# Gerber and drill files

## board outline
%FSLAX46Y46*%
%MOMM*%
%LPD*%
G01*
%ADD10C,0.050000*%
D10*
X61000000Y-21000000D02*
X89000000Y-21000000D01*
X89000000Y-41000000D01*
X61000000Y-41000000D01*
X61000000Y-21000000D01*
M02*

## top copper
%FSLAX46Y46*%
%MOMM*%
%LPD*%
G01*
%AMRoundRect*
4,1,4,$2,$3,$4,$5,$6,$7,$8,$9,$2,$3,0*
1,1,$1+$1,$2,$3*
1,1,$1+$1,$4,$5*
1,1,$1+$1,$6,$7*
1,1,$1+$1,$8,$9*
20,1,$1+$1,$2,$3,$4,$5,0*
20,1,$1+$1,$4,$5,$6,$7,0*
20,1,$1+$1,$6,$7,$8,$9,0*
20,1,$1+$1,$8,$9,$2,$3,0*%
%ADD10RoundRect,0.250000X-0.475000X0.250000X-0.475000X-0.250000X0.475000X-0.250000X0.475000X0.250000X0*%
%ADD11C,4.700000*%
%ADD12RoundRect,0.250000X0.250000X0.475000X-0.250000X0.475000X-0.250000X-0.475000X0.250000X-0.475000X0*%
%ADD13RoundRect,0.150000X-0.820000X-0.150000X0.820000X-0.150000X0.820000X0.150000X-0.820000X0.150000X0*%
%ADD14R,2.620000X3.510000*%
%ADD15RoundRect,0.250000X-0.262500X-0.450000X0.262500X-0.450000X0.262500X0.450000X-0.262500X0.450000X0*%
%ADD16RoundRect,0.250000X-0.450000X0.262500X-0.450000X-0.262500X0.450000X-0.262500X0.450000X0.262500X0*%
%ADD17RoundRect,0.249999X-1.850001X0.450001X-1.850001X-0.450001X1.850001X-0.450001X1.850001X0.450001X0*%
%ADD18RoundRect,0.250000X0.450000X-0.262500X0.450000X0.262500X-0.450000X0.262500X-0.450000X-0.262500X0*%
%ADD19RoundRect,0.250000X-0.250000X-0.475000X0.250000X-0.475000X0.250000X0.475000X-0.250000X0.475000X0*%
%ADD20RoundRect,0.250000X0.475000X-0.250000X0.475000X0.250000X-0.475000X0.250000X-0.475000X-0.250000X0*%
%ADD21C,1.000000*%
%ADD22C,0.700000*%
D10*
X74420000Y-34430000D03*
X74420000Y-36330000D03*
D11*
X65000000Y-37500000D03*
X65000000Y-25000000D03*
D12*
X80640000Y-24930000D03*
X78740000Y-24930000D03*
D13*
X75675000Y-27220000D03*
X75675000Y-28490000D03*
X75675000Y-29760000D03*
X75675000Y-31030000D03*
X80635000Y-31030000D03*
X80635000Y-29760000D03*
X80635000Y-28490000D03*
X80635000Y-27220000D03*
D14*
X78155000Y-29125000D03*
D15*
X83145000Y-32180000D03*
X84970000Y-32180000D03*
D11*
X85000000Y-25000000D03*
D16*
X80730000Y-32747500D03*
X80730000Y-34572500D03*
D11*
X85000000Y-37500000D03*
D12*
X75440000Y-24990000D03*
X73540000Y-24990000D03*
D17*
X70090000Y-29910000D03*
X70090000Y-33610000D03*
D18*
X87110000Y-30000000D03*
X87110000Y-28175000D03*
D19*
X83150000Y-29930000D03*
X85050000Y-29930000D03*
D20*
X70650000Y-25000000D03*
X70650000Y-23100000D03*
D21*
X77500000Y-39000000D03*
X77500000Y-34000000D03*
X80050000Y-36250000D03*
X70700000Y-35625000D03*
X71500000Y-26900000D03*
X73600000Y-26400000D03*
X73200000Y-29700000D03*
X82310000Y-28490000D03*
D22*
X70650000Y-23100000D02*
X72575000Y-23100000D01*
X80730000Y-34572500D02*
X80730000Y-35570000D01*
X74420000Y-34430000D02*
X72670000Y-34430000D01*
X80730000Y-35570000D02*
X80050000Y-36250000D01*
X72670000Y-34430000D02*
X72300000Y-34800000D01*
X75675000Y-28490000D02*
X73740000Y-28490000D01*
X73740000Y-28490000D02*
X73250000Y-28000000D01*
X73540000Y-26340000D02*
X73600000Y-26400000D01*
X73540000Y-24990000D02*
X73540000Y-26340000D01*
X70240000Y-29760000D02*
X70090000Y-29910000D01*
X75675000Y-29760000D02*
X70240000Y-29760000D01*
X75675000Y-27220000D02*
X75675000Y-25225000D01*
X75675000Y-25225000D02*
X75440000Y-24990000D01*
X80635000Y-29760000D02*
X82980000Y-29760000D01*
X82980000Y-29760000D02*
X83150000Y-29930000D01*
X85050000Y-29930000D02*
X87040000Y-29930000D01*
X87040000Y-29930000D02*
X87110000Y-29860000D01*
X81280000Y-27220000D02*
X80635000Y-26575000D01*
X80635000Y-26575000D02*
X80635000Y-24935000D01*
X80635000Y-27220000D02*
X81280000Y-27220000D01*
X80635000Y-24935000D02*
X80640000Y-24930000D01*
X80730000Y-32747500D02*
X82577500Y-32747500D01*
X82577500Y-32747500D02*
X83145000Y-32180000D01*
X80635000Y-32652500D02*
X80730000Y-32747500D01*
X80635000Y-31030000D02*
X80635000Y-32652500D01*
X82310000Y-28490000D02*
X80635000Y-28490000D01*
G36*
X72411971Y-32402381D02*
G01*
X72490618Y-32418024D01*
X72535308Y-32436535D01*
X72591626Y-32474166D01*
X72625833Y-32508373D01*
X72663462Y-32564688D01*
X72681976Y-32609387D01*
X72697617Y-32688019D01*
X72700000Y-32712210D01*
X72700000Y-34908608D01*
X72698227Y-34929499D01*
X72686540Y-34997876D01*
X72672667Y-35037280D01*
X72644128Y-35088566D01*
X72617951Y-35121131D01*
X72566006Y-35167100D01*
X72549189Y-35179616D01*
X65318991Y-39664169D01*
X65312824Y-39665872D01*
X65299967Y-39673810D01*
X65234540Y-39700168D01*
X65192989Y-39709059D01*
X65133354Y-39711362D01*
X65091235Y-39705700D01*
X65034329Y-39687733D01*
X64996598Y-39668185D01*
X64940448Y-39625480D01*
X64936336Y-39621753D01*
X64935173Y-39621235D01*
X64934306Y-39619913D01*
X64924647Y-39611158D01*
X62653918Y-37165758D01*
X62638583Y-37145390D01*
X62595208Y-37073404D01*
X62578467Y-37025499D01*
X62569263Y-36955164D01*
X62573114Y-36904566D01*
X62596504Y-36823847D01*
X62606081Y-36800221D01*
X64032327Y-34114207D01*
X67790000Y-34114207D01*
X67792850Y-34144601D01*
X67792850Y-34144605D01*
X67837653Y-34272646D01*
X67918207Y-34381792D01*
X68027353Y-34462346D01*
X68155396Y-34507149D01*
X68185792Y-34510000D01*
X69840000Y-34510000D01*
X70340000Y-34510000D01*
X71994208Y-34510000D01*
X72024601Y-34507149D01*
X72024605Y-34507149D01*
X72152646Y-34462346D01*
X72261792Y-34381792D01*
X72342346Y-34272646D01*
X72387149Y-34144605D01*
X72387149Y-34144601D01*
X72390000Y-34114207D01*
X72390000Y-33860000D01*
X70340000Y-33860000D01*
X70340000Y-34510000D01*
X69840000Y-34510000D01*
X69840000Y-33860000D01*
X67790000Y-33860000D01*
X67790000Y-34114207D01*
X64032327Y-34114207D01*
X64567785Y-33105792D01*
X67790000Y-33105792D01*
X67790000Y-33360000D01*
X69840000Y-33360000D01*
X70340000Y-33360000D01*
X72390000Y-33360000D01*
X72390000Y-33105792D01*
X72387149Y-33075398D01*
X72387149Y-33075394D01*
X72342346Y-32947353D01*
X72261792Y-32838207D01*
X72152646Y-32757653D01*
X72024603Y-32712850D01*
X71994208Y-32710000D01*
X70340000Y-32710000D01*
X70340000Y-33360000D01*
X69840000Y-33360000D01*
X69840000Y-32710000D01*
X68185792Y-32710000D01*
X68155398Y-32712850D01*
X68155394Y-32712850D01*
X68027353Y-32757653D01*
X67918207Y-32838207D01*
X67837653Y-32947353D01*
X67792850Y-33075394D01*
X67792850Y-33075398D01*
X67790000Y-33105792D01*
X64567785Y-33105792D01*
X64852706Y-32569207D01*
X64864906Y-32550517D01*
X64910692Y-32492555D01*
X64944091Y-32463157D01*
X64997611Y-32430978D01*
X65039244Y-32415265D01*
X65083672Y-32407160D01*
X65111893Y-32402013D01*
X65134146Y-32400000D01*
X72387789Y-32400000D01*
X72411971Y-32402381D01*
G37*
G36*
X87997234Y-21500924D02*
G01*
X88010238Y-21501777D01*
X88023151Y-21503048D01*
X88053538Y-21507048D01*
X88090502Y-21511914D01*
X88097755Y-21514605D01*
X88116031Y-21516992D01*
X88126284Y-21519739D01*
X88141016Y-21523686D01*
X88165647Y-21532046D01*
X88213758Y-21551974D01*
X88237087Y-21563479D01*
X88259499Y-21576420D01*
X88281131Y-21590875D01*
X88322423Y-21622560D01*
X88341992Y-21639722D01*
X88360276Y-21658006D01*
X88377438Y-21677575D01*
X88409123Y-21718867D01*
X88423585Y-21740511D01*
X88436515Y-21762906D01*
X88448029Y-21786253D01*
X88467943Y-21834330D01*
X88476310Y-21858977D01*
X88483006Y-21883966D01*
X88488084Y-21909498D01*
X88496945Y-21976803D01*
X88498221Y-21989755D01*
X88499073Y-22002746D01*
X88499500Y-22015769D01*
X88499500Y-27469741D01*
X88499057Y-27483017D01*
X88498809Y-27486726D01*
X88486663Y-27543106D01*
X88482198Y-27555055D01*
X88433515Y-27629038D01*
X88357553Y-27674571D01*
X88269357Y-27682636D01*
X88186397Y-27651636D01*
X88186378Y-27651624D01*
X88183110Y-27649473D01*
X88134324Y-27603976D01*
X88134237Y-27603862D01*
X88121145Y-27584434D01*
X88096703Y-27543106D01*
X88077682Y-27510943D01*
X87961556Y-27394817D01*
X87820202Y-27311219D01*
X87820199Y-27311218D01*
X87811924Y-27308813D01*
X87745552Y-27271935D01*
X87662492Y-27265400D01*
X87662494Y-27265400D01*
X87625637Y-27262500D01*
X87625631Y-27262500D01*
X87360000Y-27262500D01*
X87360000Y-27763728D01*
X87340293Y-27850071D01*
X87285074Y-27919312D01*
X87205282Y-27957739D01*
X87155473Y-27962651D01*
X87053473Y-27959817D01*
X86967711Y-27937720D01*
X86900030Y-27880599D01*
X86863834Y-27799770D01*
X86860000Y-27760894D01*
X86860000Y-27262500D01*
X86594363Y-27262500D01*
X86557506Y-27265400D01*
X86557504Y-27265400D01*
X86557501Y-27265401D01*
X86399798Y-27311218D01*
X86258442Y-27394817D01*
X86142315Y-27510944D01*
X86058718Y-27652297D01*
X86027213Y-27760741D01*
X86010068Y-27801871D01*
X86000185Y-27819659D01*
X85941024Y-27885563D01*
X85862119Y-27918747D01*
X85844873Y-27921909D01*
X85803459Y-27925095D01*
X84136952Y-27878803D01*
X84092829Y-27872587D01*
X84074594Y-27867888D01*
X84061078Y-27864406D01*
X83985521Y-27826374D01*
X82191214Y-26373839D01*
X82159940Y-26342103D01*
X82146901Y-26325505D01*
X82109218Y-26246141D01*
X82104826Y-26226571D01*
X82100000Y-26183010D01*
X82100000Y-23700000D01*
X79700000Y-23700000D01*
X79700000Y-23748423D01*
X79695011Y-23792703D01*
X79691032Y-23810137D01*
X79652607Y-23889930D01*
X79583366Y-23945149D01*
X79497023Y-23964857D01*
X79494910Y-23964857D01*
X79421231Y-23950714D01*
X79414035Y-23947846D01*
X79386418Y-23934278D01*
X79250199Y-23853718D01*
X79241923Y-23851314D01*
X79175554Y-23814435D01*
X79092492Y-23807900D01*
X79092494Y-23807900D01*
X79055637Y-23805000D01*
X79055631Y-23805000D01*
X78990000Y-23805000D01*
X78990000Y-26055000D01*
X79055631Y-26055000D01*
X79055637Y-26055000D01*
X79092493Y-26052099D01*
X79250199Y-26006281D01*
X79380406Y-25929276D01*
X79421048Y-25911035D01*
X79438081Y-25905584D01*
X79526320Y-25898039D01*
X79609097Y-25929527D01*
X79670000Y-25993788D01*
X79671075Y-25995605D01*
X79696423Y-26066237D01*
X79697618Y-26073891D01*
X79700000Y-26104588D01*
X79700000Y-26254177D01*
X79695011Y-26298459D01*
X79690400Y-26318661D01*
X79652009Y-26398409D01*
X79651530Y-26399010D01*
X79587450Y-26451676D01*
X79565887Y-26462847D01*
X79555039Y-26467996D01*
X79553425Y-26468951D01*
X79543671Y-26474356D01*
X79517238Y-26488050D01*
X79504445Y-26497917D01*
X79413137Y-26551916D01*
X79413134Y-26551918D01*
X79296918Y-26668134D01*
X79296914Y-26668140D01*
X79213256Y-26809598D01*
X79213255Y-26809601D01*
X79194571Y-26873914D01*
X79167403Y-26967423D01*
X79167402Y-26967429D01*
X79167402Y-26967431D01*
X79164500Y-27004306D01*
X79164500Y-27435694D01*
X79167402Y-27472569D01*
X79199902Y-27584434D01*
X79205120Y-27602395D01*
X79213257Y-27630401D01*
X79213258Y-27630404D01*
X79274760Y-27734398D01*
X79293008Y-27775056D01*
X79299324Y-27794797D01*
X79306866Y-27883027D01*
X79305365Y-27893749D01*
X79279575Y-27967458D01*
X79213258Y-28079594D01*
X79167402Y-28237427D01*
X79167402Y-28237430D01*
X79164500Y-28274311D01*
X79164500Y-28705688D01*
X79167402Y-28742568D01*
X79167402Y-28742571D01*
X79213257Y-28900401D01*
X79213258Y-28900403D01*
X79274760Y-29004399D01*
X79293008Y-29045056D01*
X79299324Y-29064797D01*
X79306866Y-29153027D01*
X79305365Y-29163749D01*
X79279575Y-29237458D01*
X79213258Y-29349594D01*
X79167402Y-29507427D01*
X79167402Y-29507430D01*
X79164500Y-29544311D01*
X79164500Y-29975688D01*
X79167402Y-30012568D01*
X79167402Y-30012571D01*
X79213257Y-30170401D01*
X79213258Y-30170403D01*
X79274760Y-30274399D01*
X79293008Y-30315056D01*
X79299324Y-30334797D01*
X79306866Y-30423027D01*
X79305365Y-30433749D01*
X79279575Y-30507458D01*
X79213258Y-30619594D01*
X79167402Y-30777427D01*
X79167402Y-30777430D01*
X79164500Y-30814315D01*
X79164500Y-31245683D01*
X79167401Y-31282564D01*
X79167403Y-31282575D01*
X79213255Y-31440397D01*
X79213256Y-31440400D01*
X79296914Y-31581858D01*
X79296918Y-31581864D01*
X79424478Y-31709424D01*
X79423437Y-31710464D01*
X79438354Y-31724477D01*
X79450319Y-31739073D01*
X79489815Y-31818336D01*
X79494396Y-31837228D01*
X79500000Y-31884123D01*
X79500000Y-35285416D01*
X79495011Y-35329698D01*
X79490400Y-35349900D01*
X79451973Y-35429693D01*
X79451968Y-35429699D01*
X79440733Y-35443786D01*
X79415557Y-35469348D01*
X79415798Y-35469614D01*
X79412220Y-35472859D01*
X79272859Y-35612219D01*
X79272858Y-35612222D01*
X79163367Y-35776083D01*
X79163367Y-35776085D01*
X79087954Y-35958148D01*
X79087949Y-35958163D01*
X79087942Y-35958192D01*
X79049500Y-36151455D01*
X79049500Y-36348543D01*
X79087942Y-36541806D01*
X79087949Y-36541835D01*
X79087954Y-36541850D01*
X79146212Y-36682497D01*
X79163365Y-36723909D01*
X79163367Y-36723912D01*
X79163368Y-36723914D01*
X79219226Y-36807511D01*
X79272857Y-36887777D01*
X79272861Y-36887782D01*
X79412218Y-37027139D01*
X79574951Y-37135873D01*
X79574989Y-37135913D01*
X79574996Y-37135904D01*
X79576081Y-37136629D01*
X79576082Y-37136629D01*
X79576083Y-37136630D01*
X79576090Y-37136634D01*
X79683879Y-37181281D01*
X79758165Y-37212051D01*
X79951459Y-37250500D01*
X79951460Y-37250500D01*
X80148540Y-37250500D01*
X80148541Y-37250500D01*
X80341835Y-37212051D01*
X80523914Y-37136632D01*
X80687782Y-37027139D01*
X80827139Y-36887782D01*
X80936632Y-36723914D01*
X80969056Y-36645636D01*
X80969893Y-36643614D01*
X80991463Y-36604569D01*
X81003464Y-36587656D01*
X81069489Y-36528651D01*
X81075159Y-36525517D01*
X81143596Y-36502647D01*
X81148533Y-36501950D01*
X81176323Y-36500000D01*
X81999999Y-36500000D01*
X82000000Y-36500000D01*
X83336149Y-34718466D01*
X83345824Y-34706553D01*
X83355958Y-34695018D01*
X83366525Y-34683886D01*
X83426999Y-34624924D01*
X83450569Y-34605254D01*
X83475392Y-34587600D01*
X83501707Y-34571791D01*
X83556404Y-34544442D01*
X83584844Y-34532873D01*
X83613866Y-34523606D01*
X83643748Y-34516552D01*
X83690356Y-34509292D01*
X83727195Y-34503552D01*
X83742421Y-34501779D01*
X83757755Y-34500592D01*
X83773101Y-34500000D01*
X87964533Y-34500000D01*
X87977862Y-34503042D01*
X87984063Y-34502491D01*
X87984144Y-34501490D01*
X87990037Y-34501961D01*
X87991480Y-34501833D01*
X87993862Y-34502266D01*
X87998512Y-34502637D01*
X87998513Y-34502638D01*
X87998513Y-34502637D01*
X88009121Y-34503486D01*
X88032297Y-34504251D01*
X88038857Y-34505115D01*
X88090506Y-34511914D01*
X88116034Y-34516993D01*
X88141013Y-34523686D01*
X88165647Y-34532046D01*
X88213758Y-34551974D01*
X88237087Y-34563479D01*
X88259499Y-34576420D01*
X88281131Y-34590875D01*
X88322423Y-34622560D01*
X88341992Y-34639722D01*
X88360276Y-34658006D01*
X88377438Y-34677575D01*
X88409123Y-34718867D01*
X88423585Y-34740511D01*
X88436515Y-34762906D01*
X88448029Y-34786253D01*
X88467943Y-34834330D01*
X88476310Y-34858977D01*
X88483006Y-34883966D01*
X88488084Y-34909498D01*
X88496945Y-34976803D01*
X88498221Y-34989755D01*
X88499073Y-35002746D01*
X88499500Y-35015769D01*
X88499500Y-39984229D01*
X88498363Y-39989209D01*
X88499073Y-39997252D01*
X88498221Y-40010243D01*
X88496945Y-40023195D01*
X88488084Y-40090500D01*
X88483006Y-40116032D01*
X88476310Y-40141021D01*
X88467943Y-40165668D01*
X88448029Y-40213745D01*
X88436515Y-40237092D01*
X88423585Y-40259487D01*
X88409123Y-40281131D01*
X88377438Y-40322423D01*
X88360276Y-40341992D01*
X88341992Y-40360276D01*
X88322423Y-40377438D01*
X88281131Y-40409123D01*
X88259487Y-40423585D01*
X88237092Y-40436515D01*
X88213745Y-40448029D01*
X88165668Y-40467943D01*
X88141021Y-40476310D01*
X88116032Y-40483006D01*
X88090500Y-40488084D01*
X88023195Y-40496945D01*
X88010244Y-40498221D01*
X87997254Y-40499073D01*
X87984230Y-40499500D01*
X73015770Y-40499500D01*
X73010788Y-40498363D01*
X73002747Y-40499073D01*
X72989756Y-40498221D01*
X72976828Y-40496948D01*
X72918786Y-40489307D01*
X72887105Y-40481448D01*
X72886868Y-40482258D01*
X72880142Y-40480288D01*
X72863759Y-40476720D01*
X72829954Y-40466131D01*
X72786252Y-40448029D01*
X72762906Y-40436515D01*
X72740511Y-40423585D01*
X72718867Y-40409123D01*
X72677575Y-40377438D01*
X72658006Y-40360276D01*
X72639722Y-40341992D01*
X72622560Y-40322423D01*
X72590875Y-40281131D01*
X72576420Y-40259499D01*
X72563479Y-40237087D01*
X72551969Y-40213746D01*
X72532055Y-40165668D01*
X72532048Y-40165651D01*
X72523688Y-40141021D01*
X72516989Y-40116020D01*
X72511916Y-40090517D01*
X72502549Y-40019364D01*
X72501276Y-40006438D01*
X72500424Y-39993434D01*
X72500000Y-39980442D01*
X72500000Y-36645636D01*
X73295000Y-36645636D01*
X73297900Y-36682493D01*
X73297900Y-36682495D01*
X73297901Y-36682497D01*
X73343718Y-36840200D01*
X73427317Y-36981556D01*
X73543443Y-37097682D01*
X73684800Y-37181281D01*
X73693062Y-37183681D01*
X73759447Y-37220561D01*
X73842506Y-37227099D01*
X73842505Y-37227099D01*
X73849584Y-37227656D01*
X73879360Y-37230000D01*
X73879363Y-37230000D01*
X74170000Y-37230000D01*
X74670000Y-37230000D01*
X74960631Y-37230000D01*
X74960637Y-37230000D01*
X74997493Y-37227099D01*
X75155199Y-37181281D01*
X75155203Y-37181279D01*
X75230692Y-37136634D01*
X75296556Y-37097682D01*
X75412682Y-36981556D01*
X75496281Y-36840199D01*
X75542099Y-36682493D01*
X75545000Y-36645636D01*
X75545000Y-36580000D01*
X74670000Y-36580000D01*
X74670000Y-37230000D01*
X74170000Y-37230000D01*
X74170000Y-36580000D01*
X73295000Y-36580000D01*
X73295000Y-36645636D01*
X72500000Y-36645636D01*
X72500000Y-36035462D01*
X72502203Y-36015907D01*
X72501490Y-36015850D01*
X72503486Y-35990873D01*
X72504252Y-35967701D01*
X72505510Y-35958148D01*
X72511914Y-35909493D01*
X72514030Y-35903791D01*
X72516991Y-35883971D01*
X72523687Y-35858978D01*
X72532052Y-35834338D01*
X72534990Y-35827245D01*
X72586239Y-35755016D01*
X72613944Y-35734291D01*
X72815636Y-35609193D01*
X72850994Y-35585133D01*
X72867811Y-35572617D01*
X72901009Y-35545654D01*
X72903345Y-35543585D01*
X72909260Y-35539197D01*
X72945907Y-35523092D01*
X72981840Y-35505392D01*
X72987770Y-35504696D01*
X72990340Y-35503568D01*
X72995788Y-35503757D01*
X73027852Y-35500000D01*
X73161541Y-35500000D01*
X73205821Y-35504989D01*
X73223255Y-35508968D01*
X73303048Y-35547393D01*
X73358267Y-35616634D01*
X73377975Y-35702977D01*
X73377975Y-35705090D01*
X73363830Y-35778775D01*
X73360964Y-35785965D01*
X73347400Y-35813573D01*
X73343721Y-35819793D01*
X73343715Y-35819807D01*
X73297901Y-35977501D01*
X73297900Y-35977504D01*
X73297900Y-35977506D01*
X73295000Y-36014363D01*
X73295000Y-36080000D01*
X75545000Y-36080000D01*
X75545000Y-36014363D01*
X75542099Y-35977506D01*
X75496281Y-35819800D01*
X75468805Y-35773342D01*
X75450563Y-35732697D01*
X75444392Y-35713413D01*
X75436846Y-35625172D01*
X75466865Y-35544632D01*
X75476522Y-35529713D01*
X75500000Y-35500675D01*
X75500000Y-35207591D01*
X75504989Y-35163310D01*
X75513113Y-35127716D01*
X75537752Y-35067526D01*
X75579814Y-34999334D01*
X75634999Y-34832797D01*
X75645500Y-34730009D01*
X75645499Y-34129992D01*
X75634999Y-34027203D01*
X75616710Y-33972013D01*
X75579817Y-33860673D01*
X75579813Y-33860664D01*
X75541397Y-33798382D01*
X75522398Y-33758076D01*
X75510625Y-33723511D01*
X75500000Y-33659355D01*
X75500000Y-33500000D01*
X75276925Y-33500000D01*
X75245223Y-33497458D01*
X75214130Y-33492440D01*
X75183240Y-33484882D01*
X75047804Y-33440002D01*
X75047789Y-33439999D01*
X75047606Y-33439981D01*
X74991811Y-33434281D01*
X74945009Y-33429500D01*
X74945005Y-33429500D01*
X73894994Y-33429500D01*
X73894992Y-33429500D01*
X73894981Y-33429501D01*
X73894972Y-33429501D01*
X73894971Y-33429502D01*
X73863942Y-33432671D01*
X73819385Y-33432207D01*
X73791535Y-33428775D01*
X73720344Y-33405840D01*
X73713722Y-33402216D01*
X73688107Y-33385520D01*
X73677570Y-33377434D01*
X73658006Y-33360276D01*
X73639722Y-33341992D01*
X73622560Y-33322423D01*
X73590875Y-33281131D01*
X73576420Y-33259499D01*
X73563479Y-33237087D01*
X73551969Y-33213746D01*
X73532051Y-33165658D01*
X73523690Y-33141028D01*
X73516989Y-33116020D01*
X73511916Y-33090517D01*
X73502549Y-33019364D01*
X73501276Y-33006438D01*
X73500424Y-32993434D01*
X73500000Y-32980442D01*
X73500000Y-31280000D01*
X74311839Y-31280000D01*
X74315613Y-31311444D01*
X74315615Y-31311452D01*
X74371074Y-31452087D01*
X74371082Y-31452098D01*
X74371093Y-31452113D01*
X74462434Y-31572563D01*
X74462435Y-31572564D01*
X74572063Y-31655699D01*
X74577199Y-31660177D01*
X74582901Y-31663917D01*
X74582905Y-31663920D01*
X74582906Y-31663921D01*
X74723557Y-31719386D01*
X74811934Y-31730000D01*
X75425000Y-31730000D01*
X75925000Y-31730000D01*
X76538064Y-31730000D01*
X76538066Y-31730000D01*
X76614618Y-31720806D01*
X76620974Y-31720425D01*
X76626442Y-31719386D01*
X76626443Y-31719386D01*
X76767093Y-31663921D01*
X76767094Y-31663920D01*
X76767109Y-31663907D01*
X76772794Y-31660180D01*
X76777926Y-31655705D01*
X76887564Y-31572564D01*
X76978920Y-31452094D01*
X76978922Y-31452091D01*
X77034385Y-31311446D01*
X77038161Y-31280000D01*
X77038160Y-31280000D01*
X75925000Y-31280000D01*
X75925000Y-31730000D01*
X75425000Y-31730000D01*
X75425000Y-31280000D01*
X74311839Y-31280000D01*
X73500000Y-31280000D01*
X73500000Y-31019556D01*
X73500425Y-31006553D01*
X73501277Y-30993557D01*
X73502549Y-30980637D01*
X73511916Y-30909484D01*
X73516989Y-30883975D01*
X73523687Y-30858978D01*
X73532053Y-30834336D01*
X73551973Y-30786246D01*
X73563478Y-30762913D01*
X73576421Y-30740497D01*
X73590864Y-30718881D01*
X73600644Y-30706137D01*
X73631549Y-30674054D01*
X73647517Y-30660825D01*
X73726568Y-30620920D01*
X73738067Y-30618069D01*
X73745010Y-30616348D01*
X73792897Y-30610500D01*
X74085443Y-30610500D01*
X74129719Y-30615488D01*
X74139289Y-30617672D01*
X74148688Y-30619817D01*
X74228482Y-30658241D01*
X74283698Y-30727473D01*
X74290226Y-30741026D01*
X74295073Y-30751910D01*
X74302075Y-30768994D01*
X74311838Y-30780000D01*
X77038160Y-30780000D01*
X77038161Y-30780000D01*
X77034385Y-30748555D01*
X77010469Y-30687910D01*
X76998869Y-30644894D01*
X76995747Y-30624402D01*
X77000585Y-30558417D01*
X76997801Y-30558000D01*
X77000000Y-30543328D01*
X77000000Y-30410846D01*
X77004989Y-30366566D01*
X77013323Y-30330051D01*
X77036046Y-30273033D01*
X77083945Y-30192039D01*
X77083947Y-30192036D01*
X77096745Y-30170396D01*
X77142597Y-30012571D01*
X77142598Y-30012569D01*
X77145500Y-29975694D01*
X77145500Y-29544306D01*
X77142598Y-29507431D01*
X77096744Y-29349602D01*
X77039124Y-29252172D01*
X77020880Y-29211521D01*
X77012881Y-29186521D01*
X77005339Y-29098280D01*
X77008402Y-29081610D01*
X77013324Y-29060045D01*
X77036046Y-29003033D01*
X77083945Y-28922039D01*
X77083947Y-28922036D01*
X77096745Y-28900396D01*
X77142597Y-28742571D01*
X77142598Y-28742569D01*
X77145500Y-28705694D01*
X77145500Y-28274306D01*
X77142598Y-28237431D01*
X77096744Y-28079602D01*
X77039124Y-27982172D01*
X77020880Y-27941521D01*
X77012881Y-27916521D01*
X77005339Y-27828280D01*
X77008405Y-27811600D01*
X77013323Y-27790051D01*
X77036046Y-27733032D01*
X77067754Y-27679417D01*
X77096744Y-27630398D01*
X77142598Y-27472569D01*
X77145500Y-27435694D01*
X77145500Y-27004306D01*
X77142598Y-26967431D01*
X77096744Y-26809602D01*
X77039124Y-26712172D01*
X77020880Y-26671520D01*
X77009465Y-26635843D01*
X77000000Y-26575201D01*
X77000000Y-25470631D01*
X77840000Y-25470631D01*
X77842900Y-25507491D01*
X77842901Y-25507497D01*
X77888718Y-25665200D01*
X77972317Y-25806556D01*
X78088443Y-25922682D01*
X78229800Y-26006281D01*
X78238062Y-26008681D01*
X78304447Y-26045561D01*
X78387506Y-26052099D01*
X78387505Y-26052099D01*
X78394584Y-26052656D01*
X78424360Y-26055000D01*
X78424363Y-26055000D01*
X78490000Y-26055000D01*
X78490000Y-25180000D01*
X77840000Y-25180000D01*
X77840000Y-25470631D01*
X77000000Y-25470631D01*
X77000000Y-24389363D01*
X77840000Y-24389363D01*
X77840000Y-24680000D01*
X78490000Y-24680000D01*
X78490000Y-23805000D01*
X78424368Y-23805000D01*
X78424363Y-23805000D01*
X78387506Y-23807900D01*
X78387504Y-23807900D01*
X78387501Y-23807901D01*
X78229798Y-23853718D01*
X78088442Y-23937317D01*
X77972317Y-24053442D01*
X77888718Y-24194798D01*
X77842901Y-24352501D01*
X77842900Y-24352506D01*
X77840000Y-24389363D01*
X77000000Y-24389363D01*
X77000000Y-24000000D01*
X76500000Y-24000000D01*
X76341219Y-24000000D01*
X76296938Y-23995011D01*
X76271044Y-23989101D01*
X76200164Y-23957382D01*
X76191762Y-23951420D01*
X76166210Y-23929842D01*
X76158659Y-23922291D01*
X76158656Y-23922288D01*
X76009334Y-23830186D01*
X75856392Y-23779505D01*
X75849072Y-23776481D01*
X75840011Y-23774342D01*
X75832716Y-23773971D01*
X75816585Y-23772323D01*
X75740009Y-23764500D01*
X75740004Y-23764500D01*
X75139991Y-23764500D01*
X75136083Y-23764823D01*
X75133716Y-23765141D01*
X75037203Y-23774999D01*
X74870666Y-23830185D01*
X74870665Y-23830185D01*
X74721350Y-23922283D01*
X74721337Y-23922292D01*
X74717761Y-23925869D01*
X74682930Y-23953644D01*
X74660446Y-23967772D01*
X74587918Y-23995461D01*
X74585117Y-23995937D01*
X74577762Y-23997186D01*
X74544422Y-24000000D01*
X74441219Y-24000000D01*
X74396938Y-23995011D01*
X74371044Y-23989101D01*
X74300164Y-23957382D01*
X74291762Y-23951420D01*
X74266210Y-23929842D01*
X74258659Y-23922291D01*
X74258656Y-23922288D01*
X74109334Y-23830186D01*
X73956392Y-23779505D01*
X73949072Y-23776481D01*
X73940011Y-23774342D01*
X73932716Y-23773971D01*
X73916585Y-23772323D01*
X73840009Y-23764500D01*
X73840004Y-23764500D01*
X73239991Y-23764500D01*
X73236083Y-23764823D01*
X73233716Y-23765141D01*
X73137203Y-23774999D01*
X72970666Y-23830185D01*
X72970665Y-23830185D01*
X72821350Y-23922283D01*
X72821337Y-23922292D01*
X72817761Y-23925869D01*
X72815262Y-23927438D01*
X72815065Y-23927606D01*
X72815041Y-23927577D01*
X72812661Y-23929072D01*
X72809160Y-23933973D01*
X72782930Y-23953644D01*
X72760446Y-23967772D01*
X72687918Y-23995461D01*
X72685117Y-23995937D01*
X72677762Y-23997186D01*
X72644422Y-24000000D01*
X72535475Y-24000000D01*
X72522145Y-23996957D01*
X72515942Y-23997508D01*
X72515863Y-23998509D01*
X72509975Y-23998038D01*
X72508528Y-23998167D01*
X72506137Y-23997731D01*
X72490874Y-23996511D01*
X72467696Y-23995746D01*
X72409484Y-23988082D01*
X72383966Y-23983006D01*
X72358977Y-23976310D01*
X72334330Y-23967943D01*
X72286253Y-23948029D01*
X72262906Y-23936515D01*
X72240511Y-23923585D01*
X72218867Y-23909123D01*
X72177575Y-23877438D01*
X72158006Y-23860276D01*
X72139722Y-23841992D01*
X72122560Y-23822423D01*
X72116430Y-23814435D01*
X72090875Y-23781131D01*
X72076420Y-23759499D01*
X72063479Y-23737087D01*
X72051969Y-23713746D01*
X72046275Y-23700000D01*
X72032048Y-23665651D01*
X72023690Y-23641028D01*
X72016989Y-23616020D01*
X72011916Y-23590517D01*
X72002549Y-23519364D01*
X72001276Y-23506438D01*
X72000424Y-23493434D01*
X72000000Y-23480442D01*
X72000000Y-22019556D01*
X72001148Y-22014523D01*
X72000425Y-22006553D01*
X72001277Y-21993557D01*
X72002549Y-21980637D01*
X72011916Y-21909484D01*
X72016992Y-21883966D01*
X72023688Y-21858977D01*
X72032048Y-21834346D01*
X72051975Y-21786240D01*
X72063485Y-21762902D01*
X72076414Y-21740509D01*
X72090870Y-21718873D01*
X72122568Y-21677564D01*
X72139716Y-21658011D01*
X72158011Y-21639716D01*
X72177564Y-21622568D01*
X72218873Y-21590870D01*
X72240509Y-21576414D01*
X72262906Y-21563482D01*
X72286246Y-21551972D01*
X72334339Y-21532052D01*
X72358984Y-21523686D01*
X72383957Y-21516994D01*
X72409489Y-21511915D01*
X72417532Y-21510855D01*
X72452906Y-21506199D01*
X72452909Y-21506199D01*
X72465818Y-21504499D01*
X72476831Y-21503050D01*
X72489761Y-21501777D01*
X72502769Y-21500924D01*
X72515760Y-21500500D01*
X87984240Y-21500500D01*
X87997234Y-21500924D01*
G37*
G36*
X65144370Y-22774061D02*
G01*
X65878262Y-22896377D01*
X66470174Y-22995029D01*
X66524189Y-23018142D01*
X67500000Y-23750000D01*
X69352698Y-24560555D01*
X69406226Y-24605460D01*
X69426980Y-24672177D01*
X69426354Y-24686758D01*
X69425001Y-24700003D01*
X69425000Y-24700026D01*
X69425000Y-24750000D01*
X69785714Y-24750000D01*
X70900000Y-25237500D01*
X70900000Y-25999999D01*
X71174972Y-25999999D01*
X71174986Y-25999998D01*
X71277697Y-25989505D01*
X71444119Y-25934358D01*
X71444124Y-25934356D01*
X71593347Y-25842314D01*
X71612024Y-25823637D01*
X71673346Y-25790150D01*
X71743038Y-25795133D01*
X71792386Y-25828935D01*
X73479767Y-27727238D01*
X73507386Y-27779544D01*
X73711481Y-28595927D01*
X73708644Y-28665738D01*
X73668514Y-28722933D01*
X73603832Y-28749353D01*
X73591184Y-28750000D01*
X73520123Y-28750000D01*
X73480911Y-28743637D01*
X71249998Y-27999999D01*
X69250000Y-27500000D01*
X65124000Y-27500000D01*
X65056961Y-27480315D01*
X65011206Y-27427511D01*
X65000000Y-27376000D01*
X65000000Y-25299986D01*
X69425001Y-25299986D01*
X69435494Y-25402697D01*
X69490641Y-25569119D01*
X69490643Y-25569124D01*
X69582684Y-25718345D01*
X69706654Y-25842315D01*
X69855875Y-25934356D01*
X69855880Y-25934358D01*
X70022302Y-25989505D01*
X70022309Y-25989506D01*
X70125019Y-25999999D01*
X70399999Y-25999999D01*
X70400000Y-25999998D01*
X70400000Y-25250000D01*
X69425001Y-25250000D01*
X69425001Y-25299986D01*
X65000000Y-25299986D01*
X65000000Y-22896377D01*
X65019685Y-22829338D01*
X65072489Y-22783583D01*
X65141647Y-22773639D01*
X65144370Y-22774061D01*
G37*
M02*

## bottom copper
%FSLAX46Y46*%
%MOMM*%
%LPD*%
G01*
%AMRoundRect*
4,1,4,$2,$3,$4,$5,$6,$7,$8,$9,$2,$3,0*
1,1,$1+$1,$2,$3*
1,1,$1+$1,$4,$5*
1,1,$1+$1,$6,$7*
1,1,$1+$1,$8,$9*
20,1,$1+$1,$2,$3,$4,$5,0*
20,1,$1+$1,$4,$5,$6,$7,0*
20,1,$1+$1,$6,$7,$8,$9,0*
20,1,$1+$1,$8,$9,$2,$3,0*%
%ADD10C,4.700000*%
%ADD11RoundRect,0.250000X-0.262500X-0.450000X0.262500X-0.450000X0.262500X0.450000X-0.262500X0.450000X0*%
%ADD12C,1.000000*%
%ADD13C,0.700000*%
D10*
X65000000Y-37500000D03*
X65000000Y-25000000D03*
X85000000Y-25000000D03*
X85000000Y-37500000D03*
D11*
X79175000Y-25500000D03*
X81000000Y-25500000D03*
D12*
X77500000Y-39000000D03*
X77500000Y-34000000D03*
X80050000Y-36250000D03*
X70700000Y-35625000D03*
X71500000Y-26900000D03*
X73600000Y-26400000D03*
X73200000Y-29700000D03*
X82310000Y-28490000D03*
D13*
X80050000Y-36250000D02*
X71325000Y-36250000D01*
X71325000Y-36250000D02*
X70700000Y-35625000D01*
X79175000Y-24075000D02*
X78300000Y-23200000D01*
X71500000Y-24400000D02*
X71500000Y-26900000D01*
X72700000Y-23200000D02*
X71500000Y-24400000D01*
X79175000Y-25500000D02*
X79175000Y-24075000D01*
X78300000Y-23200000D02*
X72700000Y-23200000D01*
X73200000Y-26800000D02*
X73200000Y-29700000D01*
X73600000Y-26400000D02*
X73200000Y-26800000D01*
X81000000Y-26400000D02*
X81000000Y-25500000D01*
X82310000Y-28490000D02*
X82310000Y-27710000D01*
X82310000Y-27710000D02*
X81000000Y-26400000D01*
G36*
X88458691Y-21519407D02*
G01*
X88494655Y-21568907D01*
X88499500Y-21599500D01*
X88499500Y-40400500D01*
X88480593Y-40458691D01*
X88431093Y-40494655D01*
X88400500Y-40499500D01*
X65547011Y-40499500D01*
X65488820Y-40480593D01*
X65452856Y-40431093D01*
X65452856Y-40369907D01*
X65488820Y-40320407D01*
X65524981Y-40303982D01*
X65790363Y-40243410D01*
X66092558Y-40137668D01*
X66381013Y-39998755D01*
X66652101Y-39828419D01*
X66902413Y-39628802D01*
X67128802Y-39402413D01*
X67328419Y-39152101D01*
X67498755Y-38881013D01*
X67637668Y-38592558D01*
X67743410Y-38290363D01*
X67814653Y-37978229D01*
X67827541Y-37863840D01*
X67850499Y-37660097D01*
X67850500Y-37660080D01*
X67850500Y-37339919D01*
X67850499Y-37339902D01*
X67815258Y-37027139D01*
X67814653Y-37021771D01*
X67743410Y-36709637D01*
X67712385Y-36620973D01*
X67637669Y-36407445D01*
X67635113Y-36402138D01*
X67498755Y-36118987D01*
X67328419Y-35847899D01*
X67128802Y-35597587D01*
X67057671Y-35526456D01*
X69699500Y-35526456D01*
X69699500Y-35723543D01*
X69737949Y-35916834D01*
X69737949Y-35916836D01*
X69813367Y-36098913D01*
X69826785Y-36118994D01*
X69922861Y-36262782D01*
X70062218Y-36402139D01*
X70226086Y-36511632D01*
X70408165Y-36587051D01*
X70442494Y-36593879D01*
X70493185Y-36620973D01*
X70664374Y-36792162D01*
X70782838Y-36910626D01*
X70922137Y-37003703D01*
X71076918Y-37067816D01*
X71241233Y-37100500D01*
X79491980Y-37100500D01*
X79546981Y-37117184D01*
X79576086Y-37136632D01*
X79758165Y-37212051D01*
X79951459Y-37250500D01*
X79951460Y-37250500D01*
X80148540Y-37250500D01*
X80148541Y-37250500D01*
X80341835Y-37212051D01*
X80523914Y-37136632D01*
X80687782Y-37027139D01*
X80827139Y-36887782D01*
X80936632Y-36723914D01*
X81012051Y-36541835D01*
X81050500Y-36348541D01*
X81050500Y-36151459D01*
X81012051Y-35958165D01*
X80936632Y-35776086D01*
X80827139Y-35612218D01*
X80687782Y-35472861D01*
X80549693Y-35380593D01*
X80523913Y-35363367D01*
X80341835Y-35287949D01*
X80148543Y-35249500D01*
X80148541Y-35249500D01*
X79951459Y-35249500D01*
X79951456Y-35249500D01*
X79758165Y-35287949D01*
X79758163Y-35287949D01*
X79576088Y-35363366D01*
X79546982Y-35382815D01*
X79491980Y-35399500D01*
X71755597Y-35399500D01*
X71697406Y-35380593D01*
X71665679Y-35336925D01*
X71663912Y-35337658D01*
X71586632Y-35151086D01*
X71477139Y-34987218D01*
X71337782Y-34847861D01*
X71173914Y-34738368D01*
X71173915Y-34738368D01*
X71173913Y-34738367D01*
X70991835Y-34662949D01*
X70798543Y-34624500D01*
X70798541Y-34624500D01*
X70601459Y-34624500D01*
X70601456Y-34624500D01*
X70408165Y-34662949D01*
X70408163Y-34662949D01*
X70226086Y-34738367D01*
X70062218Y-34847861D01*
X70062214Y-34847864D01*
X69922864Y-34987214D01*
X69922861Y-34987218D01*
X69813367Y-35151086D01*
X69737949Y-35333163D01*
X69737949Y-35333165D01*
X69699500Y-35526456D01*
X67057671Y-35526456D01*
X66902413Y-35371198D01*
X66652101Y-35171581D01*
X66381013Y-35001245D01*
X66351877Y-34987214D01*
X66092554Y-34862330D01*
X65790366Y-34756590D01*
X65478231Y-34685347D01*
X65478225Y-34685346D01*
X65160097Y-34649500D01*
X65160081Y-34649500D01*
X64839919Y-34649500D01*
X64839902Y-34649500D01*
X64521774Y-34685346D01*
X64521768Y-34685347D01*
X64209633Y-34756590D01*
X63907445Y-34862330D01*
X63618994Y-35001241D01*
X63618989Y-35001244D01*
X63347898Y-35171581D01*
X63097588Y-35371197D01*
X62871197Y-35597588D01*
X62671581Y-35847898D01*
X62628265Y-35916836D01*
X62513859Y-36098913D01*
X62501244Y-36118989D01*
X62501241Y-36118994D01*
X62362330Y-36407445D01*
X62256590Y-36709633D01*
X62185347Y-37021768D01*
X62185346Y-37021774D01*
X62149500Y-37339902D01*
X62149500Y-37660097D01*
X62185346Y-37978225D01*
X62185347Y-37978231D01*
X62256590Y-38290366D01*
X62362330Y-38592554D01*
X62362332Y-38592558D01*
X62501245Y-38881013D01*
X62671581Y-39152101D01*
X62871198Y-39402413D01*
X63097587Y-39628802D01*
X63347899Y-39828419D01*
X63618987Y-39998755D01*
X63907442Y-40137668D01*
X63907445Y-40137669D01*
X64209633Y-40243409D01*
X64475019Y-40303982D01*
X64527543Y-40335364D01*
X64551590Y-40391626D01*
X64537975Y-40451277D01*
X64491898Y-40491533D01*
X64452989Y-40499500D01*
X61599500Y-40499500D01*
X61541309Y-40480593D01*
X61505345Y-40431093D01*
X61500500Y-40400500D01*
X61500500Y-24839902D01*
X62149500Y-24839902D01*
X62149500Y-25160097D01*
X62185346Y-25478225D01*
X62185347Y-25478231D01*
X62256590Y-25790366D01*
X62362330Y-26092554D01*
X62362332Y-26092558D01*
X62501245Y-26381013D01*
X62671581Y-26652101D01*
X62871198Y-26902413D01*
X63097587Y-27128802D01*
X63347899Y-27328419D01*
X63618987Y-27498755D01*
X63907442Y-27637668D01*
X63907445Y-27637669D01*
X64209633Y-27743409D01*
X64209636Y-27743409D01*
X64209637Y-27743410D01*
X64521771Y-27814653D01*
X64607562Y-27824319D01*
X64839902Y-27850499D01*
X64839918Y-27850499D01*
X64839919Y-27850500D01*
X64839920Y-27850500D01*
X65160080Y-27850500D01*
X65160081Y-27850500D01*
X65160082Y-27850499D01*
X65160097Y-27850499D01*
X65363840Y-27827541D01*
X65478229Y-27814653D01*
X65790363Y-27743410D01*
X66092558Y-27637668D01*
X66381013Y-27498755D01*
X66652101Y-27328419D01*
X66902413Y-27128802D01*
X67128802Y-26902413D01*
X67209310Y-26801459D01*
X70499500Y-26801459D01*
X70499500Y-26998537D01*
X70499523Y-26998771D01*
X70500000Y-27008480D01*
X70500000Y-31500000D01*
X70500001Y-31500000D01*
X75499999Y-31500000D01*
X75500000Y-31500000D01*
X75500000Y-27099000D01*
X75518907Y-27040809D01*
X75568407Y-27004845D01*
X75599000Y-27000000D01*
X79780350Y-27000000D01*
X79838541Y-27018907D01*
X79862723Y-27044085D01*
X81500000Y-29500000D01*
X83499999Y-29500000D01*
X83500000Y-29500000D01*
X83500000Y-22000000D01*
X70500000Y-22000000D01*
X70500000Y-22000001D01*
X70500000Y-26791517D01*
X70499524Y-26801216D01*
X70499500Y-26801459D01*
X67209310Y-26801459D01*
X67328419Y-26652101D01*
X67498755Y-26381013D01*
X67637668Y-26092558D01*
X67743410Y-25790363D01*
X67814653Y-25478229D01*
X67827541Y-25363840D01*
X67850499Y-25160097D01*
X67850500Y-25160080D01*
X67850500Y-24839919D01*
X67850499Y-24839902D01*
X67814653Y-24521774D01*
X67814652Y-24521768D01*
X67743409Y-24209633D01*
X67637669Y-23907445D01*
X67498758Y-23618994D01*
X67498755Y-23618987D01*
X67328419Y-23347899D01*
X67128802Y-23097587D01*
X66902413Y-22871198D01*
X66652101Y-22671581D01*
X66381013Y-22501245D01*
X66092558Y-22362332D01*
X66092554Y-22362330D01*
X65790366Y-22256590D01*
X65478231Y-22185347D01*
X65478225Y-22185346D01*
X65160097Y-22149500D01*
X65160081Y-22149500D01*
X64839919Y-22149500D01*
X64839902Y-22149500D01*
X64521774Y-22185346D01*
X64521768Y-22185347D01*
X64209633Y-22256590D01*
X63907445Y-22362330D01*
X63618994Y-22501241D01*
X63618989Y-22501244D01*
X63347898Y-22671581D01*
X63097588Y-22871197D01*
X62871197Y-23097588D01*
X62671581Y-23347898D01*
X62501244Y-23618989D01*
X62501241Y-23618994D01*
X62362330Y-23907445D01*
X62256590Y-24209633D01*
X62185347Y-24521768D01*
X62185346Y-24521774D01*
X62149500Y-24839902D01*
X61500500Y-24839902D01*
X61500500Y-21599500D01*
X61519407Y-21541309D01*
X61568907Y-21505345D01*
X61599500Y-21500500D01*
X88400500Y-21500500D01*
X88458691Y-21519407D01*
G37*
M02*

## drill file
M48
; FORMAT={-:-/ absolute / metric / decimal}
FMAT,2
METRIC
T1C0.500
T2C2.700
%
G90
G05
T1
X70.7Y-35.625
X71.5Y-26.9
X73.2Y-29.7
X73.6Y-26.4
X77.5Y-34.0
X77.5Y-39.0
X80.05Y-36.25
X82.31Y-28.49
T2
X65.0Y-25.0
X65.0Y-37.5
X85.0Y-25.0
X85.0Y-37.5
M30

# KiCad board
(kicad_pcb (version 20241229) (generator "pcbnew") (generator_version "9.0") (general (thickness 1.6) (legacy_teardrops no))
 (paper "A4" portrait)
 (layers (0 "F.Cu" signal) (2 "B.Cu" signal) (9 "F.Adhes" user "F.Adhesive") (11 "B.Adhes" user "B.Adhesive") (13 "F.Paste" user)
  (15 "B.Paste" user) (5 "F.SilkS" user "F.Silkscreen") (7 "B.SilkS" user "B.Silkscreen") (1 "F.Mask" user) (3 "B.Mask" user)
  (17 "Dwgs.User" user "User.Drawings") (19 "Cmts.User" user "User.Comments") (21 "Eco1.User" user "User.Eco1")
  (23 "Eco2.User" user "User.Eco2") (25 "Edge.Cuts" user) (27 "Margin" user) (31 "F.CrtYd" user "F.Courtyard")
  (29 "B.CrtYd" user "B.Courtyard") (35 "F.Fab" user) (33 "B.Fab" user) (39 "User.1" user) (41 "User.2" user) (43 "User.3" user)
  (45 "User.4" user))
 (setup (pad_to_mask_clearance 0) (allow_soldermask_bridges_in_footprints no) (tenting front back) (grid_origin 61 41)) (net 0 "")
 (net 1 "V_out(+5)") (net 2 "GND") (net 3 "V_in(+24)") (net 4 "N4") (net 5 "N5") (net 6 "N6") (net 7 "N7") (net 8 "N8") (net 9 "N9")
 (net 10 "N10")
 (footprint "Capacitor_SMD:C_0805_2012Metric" (layer "F.Cu") (at 74.42 35.38 -90)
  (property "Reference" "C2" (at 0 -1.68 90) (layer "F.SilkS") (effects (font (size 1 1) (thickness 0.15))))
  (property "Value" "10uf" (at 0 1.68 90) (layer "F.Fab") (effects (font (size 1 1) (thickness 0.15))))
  (pad "1" smd roundrect (at -0.95 0 270) (size 1 1.45) (layers "F.Cu" "F.Mask" "F.Paste") (roundrect_rratio 0.25) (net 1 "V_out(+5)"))
  (pad "2" smd roundrect (at 0.95 0 270) (size 1 1.45) (layers "F.Cu" "F.Mask" "F.Paste") (roundrect_rratio 0.25) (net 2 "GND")))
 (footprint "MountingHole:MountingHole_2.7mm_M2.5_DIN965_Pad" (layer "F.Cu") (at 65 37.5)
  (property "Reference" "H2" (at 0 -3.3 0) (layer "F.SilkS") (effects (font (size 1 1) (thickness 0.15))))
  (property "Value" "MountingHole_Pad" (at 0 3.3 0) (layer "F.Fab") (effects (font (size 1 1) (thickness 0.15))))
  (pad "1" thru_hole circle (at 0 0) (size 4.7 4.7) (drill 2.7) (layers "*.Cu" "*.Mask") (remove_unused_layers no) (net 1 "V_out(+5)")
   (zone_connect 2)))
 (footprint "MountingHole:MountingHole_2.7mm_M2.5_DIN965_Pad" (layer "F.Cu") (at 65 25)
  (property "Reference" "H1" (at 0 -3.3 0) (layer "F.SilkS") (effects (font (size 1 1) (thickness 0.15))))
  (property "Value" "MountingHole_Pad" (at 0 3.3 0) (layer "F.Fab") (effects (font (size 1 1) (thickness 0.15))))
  (pad "1" thru_hole circle (at 0 0) (size 4.7 4.7) (drill 2.7) (layers "*.Cu" "*.Mask") (remove_unused_layers no) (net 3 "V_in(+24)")
   (zone_connect 2)))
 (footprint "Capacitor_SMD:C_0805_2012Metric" (layer "F.Cu") (at 79.69 24.93 180)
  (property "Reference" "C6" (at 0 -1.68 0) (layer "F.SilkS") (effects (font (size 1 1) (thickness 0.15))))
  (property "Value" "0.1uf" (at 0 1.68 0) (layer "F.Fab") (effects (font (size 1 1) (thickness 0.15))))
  (pad "1" smd roundrect (at -0.95 0 180) (size 1 1.45) (layers "F.Cu" "F.Mask" "F.Paste") (roundrect_rratio 0.25) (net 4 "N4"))
  (pad "2" smd roundrect (at 0.95 0 180) (size 1 1.45) (layers "F.Cu" "F.Mask" "F.Paste") (roundrect_rratio 0.25) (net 2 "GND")))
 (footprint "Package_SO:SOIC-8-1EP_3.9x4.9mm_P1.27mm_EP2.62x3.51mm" (layer "F.Cu") (at 78.155 29.125)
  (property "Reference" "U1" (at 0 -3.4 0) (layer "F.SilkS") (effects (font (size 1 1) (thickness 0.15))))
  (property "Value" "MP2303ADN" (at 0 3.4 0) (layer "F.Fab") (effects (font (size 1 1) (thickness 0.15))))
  (pad "" smd roundrect (at -0.655 -0.875) (size 1.06 1.41) (layers "F.Paste") (roundrect_rratio 0.235849))
  (pad "" smd roundrect (at -0.655 0.875) (size 1.06 1.41) (layers "F.Paste") (roundrect_rratio 0.235849))
  (pad "" smd roundrect (at 0.655 -0.875) (size 1.06 1.41) (layers "F.Paste") (roundrect_rratio 0.235849))
  (pad "" smd roundrect (at 0.655 0.875) (size 1.06 1.41) (layers "F.Paste") (roundrect_rratio 0.235849))
  (pad "1" smd roundrect (at -2.48 -1.905) (size 1.94 0.6) (layers "F.Cu" "F.Mask" "F.Paste") (roundrect_rratio 0.25) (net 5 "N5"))
  (pad "2" smd roundrect (at -2.48 -0.635) (size 1.94 0.6) (layers "F.Cu" "F.Mask" "F.Paste") (roundrect_rratio 0.25) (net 3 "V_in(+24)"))
  (pad "3" smd roundrect (at -2.48 0.635) (size 1.94 0.6) (layers "F.Cu" "F.Mask" "F.Paste") (roundrect_rratio 0.25) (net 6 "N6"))
  (pad "4" smd roundrect (at -2.48 1.905) (size 1.94 0.6) (layers "F.Cu" "F.Mask" "F.Paste") (roundrect_rratio 0.25) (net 2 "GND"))
  (pad "5" smd roundrect (at 2.48 1.905) (size 1.94 0.6) (layers "F.Cu" "F.Mask" "F.Paste") (roundrect_rratio 0.25) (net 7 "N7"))
  (pad "6" smd roundrect (at 2.48 0.635) (size 1.94 0.6) (layers "F.Cu" "F.Mask" "F.Paste") (roundrect_rratio 0.25) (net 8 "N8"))
  (pad "7" smd roundrect (at 2.48 -0.635) (size 1.94 0.6) (layers "F.Cu" "F.Mask" "F.Paste") (roundrect_rratio 0.25) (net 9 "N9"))
  (pad "8" smd roundrect (at 2.48 -1.905) (size 1.94 0.6) (layers "F.Cu" "F.Mask" "F.Paste") (roundrect_rratio 0.25) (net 4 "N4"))
  (pad "9" smd rect (at 0 0) (size 2.62 3.51) (layers "F.Cu" "F.Mask") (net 2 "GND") (zone_connect 2)))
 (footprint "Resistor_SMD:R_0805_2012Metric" (layer "F.Cu") (at 84.0575 32.18)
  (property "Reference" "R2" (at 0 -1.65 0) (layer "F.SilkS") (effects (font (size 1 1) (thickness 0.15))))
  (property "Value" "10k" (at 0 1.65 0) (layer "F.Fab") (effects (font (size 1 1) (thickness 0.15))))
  (pad "1" smd roundrect (at -0.9125 0) (size 1.025 1.4) (layers "F.Cu" "F.Mask" "F.Paste") (roundrect_rratio 0.243902) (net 7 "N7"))
  (pad "2" smd roundrect (at 0.9125 0) (size 1.025 1.4) (layers "F.Cu" "F.Mask" "F.Paste") (roundrect_rratio 0.243902) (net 2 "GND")))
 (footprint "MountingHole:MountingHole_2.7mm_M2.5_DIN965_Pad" (layer "F.Cu") (at 85 25)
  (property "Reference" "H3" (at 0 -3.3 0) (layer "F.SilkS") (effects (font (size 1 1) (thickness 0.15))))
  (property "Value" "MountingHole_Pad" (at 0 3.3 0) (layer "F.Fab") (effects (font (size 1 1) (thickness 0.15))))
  (pad "1" thru_hole circle (at 0 0) (size 4.7 4.7) (drill 2.7) (layers "*.Cu" "*.Mask") (remove_unused_layers no) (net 2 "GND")
   (zone_connect 2)))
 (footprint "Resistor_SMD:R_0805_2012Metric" (layer "F.Cu") (at 80.73 33.66 -90)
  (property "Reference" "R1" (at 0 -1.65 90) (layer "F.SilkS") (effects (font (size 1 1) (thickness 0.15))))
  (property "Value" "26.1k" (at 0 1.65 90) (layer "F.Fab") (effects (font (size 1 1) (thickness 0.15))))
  (pad "1" smd roundrect (at -0.9125 0 270) (size 1.025 1.4) (layers "F.Cu" "F.Mask" "F.Paste") (roundrect_rratio 0.243902) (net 7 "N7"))
  (pad "2" smd roundrect (at 0.9125 0 270) (size 1.025 1.4) (layers "F.Cu" "F.Mask" "F.Paste") (roundrect_rratio 0.243902)
   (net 1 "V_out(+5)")))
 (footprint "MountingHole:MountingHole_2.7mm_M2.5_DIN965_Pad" (layer "F.Cu") (at 85 37.5)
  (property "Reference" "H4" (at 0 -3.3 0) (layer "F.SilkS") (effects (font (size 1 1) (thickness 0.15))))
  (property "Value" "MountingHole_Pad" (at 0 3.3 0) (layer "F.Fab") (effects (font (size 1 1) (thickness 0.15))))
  (pad "1" thru_hole circle (at 0 0) (size 4.7 4.7) (drill 2.7) (layers "*.Cu" "*.Mask") (remove_unused_layers no) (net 2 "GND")
   (zone_connect 2)))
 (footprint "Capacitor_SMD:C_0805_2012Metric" (layer "F.Cu") (at 74.49 24.99 180)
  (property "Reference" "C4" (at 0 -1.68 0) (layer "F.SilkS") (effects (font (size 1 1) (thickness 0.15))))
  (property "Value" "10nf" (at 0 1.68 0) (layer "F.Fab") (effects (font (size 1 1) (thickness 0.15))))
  (pad "1" smd roundrect (at -0.95 0 180) (size 1 1.45) (layers "F.Cu" "F.Mask" "F.Paste") (roundrect_rratio 0.25) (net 5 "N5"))
  (pad "2" smd roundrect (at 0.95 0 180) (size 1 1.45) (layers "F.Cu" "F.Mask" "F.Paste") (roundrect_rratio 0.25) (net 6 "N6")))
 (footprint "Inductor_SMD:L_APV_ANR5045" (layer "F.Cu") (at 70.09 31.76 -90)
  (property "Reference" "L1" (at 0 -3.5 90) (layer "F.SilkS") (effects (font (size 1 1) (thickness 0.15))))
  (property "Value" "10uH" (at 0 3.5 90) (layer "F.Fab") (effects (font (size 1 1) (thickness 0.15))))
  (pad "1" smd roundrect (at -1.85 0 270) (size 1.4 4.2) (layers "F.Cu" "F.Mask" "F.Paste") (roundrect_rratio 0.178571) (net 6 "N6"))
  (pad "2" smd roundrect (at 1.85 0 270) (size 1.4 4.2) (layers "F.Cu" "F.Mask" "F.Paste") (roundrect_rratio 0.178571) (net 1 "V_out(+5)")))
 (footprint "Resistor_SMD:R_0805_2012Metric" (layer "F.Cu") (at 87.11 29.0875 90)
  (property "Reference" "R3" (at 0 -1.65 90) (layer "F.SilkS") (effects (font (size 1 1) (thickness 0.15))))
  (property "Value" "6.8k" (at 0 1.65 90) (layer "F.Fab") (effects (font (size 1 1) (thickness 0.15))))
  (pad "1" smd roundrect (at -0.9125 0 90) (size 1.025 1.4) (layers "F.Cu" "F.Mask" "F.Paste") (roundrect_rratio 0.243902) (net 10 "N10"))
  (pad "2" smd roundrect (at 0.9125 0 90) (size 1.025 1.4) (layers "F.Cu" "F.Mask" "F.Paste") (roundrect_rratio 0.243902) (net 2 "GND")))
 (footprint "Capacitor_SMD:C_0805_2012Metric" (layer "F.Cu") (at 84.1 29.93)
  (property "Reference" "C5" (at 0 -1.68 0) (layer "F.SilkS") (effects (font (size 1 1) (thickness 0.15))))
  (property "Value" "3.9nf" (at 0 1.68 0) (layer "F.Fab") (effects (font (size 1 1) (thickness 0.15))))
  (pad "1" smd roundrect (at -0.95 0) (size 1 1.45) (layers "F.Cu" "F.Mask" "F.Paste") (roundrect_rratio 0.25) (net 8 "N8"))
  (pad "2" smd roundrect (at 0.95 0) (size 1 1.45) (layers "F.Cu" "F.Mask" "F.Paste") (roundrect_rratio 0.25) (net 10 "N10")))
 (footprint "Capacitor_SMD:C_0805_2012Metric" (layer "F.Cu") (at 70.65 24.05 90)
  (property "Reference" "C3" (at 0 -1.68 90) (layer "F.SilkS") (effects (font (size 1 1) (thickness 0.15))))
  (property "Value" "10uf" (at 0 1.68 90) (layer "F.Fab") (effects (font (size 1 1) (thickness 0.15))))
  (pad "1" smd roundrect (at -0.95 0 90) (size 1 1.45) (layers "F.Cu" "F.Mask" "F.Paste") (roundrect_rratio 0.25) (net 3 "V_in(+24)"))
  (pad "2" smd roundrect (at 0.95 0 90) (size 1 1.45) (layers "F.Cu" "F.Mask" "F.Paste") (roundrect_rratio 0.25) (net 2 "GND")))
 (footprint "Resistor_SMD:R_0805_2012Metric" (layer "B.Cu") (at 80.0875 25.5)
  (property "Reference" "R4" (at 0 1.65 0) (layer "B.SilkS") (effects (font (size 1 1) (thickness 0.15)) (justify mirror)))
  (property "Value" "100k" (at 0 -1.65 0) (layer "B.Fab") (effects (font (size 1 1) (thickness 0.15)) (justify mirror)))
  (pad "1" smd roundrect (at -0.9125 0) (size 1.025 1.4) (layers "B.Cu" "B.Mask" "B.Paste") (roundrect_rratio 0.243902) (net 3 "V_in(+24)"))
  (pad "2" smd roundrect (at 0.9125 0) (size 1.025 1.4) (layers "B.Cu" "B.Mask" "B.Paste") (roundrect_rratio 0.243902) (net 9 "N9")))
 (gr_rect (start 61 21) (end 89 41) (stroke (width 0.05) (type default)) (fill no) (layer "Edge.Cuts"))
 (segment (start 70.65 23.1) (end 72.575 23.1) (width 0.7) (layer "F.Cu") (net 2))
 (via (at 77.5 39) (size 1) (drill 0.5) (layers "F.Cu" "B.Cu") (free yes) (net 2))
 (via (at 77.5 34) (size 1) (drill 0.5) (layers "F.Cu" "B.Cu") (free yes) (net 2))
 (segment (start 80.73 34.5725) (end 80.73 35.57) (width 0.7) (layer "F.Cu") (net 1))
 (segment (start 74.42 34.43) (end 72.67 34.43) (width 0.7) (layer "F.Cu") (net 1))
 (segment (start 80.73 35.57) (end 80.05 36.25) (width 0.7) (layer "F.Cu") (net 1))
 (segment (start 72.67 34.43) (end 72.3 34.8) (width 0.7) (layer "F.Cu") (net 1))
 (via (at 80.05 36.25) (size 1) (drill 0.5) (layers "F.Cu" "B.Cu") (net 1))
 (via (at 70.7 35.625) (size 1) (drill 0.5) (layers "F.Cu" "B.Cu") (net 1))
 (segment (start 80.05 36.25) (end 71.325 36.25) (width 0.7) (layer "B.Cu") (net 1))
 (segment (start 71.325 36.25) (end 70.7 35.625) (width 0.7) (layer "B.Cu") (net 1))
 (segment (start 75.675 28.49) (end 73.74 28.49) (width 0.7) (layer "F.Cu") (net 3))
 (segment (start 73.74 28.49) (end 73.25 28) (width 0.7) (layer "F.Cu") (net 3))
 (via (at 71.5 26.9) (size 1) (drill 0.5) (layers "F.Cu" "B.Cu") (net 3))
 (segment (start 79.175 24.075) (end 78.3 23.2) (width 0.7) (layer "B.Cu") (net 3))
 (segment (start 71.5 24.4) (end 71.5 26.9) (width 0.7) (layer "B.Cu") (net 3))
 (segment (start 72.7 23.2) (end 71.5 24.4) (width 0.7) (layer "B.Cu") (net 3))
 (segment (start 79.175 25.5) (end 79.175 24.075) (width 0.7) (layer "B.Cu") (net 3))
 (segment (start 78.3 23.2) (end 72.7 23.2) (width 0.7) (layer "B.Cu") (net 3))
 (segment (start 73.54 26.34) (end 73.6 26.4) (width 0.7) (layer "F.Cu") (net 6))
 (segment (start 73.54 24.99) (end 73.54 26.34) (width 0.7) (layer "F.Cu") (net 6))
 (segment (start 70.24 29.76) (end 70.09 29.91) (width 0.7) (layer "F.Cu") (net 6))
 (segment (start 75.675 29.76) (end 70.24 29.76) (width 0.7) (layer "F.Cu") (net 6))
 (via (at 73.6 26.4) (size 1) (drill 0.5) (layers "F.Cu" "B.Cu") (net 6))
 (via (at 73.2 29.7) (size 1) (drill 0.5) (layers "F.Cu" "B.Cu") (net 6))
 (segment (start 73.2 26.8) (end 73.2 29.7) (width 0.7) (layer "B.Cu") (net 6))
 (segment (start 73.6 26.4) (end 73.2 26.8) (width 0.7) (layer "B.Cu") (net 6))
 (segment (start 75.675 27.22) (end 75.675 25.225) (width 0.7) (layer "F.Cu") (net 5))
 (segment (start 75.675 25.225) (end 75.44 24.99) (width 0.7) (layer "F.Cu") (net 5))
 (segment (start 80.635 29.76) (end 82.98 29.76) (width 0.7) (layer "F.Cu") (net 8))
 (segment (start 82.98 29.76) (end 83.15 29.93) (width 0.7) (layer "F.Cu") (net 8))
 (segment (start 85.05 29.93) (end 87.04 29.93) (width 0.7) (layer "F.Cu") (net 10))
 (segment (start 87.04 29.93) (end 87.11 29.86) (width 0.7) (layer "F.Cu") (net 10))
 (segment (start 81.28 27.22) (end 80.635 26.575) (width 0.7) (layer "F.Cu") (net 4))
 (segment (start 80.635 26.575) (end 80.635 24.935) (width 0.7) (layer "F.Cu") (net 4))
 (segment (start 80.635 27.22) (end 81.28 27.22) (width 0.7) (layer "F.Cu") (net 4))
 (segment (start 80.635 24.935) (end 80.64 24.93) (width 0.7) (layer "F.Cu") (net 4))
 (segment (start 80.73 32.7475) (end 82.5775 32.7475) (width 0.7) (layer "F.Cu") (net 7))
 (segment (start 82.5775 32.7475) (end 83.145 32.18) (width 0.7) (layer "F.Cu") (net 7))
 (segment (start 80.635 32.6525) (end 80.73 32.7475) (width 0.7) (layer "F.Cu") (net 7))
 (segment (start 80.635 31.03) (end 80.635 32.6525) (width 0.7) (layer "F.Cu") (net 7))
 (segment (start 82.31 28.49) (end 80.635 28.49) (width 0.7) (layer "F.Cu") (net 9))
 (via (at 82.31 28.49) (size 1) (drill 0.5) (layers "F.Cu" "B.Cu") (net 9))
 (segment (start 81 26.4) (end 81 25.5) (width 0.7) (layer "B.Cu") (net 9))
 (segment (start 82.31 28.49) (end 82.31 27.71) (width 0.7) (layer "B.Cu") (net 9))
 (segment (start 82.31 27.71) (end 81 26.4) (width 0.7) (layer "B.Cu") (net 9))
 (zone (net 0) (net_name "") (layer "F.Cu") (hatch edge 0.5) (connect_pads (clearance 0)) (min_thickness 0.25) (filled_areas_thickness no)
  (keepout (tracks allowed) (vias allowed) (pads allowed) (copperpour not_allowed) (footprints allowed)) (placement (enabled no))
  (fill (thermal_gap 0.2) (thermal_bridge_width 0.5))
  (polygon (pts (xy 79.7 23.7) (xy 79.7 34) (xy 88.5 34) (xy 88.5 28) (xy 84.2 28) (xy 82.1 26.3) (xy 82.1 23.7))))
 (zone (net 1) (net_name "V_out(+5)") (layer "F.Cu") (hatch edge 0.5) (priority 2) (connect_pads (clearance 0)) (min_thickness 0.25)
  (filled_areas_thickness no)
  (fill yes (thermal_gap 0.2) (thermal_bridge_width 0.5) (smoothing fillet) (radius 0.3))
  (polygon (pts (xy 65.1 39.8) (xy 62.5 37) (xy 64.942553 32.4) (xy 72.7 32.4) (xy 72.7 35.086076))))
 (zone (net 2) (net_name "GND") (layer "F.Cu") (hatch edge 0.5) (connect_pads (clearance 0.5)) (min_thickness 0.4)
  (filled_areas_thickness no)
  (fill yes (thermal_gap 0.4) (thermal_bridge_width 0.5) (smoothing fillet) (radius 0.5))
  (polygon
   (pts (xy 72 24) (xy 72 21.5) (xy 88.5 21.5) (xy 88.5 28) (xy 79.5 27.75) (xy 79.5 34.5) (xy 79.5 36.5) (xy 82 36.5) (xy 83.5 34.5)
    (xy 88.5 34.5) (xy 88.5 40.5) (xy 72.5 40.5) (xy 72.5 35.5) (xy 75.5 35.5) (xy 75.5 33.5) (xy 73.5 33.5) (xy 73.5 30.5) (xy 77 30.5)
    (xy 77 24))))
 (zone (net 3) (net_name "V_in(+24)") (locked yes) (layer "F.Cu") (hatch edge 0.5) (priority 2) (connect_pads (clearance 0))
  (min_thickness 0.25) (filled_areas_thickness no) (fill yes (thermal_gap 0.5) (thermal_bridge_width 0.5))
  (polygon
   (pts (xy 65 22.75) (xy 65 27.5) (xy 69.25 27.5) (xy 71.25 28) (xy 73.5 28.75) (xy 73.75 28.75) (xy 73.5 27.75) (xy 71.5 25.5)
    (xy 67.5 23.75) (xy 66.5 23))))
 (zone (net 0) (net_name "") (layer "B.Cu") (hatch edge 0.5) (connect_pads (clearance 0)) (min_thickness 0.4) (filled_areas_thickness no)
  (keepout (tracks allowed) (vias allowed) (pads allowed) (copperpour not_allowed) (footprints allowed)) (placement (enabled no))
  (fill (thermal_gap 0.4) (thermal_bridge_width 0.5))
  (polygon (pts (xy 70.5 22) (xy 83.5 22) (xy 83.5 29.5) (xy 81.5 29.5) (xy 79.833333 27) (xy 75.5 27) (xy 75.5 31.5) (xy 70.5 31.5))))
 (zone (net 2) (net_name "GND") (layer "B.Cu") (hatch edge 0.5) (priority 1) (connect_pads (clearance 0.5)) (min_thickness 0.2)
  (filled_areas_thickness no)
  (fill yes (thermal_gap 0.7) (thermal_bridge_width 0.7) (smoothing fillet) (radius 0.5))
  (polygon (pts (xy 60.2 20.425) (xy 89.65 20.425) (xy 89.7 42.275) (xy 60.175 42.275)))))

